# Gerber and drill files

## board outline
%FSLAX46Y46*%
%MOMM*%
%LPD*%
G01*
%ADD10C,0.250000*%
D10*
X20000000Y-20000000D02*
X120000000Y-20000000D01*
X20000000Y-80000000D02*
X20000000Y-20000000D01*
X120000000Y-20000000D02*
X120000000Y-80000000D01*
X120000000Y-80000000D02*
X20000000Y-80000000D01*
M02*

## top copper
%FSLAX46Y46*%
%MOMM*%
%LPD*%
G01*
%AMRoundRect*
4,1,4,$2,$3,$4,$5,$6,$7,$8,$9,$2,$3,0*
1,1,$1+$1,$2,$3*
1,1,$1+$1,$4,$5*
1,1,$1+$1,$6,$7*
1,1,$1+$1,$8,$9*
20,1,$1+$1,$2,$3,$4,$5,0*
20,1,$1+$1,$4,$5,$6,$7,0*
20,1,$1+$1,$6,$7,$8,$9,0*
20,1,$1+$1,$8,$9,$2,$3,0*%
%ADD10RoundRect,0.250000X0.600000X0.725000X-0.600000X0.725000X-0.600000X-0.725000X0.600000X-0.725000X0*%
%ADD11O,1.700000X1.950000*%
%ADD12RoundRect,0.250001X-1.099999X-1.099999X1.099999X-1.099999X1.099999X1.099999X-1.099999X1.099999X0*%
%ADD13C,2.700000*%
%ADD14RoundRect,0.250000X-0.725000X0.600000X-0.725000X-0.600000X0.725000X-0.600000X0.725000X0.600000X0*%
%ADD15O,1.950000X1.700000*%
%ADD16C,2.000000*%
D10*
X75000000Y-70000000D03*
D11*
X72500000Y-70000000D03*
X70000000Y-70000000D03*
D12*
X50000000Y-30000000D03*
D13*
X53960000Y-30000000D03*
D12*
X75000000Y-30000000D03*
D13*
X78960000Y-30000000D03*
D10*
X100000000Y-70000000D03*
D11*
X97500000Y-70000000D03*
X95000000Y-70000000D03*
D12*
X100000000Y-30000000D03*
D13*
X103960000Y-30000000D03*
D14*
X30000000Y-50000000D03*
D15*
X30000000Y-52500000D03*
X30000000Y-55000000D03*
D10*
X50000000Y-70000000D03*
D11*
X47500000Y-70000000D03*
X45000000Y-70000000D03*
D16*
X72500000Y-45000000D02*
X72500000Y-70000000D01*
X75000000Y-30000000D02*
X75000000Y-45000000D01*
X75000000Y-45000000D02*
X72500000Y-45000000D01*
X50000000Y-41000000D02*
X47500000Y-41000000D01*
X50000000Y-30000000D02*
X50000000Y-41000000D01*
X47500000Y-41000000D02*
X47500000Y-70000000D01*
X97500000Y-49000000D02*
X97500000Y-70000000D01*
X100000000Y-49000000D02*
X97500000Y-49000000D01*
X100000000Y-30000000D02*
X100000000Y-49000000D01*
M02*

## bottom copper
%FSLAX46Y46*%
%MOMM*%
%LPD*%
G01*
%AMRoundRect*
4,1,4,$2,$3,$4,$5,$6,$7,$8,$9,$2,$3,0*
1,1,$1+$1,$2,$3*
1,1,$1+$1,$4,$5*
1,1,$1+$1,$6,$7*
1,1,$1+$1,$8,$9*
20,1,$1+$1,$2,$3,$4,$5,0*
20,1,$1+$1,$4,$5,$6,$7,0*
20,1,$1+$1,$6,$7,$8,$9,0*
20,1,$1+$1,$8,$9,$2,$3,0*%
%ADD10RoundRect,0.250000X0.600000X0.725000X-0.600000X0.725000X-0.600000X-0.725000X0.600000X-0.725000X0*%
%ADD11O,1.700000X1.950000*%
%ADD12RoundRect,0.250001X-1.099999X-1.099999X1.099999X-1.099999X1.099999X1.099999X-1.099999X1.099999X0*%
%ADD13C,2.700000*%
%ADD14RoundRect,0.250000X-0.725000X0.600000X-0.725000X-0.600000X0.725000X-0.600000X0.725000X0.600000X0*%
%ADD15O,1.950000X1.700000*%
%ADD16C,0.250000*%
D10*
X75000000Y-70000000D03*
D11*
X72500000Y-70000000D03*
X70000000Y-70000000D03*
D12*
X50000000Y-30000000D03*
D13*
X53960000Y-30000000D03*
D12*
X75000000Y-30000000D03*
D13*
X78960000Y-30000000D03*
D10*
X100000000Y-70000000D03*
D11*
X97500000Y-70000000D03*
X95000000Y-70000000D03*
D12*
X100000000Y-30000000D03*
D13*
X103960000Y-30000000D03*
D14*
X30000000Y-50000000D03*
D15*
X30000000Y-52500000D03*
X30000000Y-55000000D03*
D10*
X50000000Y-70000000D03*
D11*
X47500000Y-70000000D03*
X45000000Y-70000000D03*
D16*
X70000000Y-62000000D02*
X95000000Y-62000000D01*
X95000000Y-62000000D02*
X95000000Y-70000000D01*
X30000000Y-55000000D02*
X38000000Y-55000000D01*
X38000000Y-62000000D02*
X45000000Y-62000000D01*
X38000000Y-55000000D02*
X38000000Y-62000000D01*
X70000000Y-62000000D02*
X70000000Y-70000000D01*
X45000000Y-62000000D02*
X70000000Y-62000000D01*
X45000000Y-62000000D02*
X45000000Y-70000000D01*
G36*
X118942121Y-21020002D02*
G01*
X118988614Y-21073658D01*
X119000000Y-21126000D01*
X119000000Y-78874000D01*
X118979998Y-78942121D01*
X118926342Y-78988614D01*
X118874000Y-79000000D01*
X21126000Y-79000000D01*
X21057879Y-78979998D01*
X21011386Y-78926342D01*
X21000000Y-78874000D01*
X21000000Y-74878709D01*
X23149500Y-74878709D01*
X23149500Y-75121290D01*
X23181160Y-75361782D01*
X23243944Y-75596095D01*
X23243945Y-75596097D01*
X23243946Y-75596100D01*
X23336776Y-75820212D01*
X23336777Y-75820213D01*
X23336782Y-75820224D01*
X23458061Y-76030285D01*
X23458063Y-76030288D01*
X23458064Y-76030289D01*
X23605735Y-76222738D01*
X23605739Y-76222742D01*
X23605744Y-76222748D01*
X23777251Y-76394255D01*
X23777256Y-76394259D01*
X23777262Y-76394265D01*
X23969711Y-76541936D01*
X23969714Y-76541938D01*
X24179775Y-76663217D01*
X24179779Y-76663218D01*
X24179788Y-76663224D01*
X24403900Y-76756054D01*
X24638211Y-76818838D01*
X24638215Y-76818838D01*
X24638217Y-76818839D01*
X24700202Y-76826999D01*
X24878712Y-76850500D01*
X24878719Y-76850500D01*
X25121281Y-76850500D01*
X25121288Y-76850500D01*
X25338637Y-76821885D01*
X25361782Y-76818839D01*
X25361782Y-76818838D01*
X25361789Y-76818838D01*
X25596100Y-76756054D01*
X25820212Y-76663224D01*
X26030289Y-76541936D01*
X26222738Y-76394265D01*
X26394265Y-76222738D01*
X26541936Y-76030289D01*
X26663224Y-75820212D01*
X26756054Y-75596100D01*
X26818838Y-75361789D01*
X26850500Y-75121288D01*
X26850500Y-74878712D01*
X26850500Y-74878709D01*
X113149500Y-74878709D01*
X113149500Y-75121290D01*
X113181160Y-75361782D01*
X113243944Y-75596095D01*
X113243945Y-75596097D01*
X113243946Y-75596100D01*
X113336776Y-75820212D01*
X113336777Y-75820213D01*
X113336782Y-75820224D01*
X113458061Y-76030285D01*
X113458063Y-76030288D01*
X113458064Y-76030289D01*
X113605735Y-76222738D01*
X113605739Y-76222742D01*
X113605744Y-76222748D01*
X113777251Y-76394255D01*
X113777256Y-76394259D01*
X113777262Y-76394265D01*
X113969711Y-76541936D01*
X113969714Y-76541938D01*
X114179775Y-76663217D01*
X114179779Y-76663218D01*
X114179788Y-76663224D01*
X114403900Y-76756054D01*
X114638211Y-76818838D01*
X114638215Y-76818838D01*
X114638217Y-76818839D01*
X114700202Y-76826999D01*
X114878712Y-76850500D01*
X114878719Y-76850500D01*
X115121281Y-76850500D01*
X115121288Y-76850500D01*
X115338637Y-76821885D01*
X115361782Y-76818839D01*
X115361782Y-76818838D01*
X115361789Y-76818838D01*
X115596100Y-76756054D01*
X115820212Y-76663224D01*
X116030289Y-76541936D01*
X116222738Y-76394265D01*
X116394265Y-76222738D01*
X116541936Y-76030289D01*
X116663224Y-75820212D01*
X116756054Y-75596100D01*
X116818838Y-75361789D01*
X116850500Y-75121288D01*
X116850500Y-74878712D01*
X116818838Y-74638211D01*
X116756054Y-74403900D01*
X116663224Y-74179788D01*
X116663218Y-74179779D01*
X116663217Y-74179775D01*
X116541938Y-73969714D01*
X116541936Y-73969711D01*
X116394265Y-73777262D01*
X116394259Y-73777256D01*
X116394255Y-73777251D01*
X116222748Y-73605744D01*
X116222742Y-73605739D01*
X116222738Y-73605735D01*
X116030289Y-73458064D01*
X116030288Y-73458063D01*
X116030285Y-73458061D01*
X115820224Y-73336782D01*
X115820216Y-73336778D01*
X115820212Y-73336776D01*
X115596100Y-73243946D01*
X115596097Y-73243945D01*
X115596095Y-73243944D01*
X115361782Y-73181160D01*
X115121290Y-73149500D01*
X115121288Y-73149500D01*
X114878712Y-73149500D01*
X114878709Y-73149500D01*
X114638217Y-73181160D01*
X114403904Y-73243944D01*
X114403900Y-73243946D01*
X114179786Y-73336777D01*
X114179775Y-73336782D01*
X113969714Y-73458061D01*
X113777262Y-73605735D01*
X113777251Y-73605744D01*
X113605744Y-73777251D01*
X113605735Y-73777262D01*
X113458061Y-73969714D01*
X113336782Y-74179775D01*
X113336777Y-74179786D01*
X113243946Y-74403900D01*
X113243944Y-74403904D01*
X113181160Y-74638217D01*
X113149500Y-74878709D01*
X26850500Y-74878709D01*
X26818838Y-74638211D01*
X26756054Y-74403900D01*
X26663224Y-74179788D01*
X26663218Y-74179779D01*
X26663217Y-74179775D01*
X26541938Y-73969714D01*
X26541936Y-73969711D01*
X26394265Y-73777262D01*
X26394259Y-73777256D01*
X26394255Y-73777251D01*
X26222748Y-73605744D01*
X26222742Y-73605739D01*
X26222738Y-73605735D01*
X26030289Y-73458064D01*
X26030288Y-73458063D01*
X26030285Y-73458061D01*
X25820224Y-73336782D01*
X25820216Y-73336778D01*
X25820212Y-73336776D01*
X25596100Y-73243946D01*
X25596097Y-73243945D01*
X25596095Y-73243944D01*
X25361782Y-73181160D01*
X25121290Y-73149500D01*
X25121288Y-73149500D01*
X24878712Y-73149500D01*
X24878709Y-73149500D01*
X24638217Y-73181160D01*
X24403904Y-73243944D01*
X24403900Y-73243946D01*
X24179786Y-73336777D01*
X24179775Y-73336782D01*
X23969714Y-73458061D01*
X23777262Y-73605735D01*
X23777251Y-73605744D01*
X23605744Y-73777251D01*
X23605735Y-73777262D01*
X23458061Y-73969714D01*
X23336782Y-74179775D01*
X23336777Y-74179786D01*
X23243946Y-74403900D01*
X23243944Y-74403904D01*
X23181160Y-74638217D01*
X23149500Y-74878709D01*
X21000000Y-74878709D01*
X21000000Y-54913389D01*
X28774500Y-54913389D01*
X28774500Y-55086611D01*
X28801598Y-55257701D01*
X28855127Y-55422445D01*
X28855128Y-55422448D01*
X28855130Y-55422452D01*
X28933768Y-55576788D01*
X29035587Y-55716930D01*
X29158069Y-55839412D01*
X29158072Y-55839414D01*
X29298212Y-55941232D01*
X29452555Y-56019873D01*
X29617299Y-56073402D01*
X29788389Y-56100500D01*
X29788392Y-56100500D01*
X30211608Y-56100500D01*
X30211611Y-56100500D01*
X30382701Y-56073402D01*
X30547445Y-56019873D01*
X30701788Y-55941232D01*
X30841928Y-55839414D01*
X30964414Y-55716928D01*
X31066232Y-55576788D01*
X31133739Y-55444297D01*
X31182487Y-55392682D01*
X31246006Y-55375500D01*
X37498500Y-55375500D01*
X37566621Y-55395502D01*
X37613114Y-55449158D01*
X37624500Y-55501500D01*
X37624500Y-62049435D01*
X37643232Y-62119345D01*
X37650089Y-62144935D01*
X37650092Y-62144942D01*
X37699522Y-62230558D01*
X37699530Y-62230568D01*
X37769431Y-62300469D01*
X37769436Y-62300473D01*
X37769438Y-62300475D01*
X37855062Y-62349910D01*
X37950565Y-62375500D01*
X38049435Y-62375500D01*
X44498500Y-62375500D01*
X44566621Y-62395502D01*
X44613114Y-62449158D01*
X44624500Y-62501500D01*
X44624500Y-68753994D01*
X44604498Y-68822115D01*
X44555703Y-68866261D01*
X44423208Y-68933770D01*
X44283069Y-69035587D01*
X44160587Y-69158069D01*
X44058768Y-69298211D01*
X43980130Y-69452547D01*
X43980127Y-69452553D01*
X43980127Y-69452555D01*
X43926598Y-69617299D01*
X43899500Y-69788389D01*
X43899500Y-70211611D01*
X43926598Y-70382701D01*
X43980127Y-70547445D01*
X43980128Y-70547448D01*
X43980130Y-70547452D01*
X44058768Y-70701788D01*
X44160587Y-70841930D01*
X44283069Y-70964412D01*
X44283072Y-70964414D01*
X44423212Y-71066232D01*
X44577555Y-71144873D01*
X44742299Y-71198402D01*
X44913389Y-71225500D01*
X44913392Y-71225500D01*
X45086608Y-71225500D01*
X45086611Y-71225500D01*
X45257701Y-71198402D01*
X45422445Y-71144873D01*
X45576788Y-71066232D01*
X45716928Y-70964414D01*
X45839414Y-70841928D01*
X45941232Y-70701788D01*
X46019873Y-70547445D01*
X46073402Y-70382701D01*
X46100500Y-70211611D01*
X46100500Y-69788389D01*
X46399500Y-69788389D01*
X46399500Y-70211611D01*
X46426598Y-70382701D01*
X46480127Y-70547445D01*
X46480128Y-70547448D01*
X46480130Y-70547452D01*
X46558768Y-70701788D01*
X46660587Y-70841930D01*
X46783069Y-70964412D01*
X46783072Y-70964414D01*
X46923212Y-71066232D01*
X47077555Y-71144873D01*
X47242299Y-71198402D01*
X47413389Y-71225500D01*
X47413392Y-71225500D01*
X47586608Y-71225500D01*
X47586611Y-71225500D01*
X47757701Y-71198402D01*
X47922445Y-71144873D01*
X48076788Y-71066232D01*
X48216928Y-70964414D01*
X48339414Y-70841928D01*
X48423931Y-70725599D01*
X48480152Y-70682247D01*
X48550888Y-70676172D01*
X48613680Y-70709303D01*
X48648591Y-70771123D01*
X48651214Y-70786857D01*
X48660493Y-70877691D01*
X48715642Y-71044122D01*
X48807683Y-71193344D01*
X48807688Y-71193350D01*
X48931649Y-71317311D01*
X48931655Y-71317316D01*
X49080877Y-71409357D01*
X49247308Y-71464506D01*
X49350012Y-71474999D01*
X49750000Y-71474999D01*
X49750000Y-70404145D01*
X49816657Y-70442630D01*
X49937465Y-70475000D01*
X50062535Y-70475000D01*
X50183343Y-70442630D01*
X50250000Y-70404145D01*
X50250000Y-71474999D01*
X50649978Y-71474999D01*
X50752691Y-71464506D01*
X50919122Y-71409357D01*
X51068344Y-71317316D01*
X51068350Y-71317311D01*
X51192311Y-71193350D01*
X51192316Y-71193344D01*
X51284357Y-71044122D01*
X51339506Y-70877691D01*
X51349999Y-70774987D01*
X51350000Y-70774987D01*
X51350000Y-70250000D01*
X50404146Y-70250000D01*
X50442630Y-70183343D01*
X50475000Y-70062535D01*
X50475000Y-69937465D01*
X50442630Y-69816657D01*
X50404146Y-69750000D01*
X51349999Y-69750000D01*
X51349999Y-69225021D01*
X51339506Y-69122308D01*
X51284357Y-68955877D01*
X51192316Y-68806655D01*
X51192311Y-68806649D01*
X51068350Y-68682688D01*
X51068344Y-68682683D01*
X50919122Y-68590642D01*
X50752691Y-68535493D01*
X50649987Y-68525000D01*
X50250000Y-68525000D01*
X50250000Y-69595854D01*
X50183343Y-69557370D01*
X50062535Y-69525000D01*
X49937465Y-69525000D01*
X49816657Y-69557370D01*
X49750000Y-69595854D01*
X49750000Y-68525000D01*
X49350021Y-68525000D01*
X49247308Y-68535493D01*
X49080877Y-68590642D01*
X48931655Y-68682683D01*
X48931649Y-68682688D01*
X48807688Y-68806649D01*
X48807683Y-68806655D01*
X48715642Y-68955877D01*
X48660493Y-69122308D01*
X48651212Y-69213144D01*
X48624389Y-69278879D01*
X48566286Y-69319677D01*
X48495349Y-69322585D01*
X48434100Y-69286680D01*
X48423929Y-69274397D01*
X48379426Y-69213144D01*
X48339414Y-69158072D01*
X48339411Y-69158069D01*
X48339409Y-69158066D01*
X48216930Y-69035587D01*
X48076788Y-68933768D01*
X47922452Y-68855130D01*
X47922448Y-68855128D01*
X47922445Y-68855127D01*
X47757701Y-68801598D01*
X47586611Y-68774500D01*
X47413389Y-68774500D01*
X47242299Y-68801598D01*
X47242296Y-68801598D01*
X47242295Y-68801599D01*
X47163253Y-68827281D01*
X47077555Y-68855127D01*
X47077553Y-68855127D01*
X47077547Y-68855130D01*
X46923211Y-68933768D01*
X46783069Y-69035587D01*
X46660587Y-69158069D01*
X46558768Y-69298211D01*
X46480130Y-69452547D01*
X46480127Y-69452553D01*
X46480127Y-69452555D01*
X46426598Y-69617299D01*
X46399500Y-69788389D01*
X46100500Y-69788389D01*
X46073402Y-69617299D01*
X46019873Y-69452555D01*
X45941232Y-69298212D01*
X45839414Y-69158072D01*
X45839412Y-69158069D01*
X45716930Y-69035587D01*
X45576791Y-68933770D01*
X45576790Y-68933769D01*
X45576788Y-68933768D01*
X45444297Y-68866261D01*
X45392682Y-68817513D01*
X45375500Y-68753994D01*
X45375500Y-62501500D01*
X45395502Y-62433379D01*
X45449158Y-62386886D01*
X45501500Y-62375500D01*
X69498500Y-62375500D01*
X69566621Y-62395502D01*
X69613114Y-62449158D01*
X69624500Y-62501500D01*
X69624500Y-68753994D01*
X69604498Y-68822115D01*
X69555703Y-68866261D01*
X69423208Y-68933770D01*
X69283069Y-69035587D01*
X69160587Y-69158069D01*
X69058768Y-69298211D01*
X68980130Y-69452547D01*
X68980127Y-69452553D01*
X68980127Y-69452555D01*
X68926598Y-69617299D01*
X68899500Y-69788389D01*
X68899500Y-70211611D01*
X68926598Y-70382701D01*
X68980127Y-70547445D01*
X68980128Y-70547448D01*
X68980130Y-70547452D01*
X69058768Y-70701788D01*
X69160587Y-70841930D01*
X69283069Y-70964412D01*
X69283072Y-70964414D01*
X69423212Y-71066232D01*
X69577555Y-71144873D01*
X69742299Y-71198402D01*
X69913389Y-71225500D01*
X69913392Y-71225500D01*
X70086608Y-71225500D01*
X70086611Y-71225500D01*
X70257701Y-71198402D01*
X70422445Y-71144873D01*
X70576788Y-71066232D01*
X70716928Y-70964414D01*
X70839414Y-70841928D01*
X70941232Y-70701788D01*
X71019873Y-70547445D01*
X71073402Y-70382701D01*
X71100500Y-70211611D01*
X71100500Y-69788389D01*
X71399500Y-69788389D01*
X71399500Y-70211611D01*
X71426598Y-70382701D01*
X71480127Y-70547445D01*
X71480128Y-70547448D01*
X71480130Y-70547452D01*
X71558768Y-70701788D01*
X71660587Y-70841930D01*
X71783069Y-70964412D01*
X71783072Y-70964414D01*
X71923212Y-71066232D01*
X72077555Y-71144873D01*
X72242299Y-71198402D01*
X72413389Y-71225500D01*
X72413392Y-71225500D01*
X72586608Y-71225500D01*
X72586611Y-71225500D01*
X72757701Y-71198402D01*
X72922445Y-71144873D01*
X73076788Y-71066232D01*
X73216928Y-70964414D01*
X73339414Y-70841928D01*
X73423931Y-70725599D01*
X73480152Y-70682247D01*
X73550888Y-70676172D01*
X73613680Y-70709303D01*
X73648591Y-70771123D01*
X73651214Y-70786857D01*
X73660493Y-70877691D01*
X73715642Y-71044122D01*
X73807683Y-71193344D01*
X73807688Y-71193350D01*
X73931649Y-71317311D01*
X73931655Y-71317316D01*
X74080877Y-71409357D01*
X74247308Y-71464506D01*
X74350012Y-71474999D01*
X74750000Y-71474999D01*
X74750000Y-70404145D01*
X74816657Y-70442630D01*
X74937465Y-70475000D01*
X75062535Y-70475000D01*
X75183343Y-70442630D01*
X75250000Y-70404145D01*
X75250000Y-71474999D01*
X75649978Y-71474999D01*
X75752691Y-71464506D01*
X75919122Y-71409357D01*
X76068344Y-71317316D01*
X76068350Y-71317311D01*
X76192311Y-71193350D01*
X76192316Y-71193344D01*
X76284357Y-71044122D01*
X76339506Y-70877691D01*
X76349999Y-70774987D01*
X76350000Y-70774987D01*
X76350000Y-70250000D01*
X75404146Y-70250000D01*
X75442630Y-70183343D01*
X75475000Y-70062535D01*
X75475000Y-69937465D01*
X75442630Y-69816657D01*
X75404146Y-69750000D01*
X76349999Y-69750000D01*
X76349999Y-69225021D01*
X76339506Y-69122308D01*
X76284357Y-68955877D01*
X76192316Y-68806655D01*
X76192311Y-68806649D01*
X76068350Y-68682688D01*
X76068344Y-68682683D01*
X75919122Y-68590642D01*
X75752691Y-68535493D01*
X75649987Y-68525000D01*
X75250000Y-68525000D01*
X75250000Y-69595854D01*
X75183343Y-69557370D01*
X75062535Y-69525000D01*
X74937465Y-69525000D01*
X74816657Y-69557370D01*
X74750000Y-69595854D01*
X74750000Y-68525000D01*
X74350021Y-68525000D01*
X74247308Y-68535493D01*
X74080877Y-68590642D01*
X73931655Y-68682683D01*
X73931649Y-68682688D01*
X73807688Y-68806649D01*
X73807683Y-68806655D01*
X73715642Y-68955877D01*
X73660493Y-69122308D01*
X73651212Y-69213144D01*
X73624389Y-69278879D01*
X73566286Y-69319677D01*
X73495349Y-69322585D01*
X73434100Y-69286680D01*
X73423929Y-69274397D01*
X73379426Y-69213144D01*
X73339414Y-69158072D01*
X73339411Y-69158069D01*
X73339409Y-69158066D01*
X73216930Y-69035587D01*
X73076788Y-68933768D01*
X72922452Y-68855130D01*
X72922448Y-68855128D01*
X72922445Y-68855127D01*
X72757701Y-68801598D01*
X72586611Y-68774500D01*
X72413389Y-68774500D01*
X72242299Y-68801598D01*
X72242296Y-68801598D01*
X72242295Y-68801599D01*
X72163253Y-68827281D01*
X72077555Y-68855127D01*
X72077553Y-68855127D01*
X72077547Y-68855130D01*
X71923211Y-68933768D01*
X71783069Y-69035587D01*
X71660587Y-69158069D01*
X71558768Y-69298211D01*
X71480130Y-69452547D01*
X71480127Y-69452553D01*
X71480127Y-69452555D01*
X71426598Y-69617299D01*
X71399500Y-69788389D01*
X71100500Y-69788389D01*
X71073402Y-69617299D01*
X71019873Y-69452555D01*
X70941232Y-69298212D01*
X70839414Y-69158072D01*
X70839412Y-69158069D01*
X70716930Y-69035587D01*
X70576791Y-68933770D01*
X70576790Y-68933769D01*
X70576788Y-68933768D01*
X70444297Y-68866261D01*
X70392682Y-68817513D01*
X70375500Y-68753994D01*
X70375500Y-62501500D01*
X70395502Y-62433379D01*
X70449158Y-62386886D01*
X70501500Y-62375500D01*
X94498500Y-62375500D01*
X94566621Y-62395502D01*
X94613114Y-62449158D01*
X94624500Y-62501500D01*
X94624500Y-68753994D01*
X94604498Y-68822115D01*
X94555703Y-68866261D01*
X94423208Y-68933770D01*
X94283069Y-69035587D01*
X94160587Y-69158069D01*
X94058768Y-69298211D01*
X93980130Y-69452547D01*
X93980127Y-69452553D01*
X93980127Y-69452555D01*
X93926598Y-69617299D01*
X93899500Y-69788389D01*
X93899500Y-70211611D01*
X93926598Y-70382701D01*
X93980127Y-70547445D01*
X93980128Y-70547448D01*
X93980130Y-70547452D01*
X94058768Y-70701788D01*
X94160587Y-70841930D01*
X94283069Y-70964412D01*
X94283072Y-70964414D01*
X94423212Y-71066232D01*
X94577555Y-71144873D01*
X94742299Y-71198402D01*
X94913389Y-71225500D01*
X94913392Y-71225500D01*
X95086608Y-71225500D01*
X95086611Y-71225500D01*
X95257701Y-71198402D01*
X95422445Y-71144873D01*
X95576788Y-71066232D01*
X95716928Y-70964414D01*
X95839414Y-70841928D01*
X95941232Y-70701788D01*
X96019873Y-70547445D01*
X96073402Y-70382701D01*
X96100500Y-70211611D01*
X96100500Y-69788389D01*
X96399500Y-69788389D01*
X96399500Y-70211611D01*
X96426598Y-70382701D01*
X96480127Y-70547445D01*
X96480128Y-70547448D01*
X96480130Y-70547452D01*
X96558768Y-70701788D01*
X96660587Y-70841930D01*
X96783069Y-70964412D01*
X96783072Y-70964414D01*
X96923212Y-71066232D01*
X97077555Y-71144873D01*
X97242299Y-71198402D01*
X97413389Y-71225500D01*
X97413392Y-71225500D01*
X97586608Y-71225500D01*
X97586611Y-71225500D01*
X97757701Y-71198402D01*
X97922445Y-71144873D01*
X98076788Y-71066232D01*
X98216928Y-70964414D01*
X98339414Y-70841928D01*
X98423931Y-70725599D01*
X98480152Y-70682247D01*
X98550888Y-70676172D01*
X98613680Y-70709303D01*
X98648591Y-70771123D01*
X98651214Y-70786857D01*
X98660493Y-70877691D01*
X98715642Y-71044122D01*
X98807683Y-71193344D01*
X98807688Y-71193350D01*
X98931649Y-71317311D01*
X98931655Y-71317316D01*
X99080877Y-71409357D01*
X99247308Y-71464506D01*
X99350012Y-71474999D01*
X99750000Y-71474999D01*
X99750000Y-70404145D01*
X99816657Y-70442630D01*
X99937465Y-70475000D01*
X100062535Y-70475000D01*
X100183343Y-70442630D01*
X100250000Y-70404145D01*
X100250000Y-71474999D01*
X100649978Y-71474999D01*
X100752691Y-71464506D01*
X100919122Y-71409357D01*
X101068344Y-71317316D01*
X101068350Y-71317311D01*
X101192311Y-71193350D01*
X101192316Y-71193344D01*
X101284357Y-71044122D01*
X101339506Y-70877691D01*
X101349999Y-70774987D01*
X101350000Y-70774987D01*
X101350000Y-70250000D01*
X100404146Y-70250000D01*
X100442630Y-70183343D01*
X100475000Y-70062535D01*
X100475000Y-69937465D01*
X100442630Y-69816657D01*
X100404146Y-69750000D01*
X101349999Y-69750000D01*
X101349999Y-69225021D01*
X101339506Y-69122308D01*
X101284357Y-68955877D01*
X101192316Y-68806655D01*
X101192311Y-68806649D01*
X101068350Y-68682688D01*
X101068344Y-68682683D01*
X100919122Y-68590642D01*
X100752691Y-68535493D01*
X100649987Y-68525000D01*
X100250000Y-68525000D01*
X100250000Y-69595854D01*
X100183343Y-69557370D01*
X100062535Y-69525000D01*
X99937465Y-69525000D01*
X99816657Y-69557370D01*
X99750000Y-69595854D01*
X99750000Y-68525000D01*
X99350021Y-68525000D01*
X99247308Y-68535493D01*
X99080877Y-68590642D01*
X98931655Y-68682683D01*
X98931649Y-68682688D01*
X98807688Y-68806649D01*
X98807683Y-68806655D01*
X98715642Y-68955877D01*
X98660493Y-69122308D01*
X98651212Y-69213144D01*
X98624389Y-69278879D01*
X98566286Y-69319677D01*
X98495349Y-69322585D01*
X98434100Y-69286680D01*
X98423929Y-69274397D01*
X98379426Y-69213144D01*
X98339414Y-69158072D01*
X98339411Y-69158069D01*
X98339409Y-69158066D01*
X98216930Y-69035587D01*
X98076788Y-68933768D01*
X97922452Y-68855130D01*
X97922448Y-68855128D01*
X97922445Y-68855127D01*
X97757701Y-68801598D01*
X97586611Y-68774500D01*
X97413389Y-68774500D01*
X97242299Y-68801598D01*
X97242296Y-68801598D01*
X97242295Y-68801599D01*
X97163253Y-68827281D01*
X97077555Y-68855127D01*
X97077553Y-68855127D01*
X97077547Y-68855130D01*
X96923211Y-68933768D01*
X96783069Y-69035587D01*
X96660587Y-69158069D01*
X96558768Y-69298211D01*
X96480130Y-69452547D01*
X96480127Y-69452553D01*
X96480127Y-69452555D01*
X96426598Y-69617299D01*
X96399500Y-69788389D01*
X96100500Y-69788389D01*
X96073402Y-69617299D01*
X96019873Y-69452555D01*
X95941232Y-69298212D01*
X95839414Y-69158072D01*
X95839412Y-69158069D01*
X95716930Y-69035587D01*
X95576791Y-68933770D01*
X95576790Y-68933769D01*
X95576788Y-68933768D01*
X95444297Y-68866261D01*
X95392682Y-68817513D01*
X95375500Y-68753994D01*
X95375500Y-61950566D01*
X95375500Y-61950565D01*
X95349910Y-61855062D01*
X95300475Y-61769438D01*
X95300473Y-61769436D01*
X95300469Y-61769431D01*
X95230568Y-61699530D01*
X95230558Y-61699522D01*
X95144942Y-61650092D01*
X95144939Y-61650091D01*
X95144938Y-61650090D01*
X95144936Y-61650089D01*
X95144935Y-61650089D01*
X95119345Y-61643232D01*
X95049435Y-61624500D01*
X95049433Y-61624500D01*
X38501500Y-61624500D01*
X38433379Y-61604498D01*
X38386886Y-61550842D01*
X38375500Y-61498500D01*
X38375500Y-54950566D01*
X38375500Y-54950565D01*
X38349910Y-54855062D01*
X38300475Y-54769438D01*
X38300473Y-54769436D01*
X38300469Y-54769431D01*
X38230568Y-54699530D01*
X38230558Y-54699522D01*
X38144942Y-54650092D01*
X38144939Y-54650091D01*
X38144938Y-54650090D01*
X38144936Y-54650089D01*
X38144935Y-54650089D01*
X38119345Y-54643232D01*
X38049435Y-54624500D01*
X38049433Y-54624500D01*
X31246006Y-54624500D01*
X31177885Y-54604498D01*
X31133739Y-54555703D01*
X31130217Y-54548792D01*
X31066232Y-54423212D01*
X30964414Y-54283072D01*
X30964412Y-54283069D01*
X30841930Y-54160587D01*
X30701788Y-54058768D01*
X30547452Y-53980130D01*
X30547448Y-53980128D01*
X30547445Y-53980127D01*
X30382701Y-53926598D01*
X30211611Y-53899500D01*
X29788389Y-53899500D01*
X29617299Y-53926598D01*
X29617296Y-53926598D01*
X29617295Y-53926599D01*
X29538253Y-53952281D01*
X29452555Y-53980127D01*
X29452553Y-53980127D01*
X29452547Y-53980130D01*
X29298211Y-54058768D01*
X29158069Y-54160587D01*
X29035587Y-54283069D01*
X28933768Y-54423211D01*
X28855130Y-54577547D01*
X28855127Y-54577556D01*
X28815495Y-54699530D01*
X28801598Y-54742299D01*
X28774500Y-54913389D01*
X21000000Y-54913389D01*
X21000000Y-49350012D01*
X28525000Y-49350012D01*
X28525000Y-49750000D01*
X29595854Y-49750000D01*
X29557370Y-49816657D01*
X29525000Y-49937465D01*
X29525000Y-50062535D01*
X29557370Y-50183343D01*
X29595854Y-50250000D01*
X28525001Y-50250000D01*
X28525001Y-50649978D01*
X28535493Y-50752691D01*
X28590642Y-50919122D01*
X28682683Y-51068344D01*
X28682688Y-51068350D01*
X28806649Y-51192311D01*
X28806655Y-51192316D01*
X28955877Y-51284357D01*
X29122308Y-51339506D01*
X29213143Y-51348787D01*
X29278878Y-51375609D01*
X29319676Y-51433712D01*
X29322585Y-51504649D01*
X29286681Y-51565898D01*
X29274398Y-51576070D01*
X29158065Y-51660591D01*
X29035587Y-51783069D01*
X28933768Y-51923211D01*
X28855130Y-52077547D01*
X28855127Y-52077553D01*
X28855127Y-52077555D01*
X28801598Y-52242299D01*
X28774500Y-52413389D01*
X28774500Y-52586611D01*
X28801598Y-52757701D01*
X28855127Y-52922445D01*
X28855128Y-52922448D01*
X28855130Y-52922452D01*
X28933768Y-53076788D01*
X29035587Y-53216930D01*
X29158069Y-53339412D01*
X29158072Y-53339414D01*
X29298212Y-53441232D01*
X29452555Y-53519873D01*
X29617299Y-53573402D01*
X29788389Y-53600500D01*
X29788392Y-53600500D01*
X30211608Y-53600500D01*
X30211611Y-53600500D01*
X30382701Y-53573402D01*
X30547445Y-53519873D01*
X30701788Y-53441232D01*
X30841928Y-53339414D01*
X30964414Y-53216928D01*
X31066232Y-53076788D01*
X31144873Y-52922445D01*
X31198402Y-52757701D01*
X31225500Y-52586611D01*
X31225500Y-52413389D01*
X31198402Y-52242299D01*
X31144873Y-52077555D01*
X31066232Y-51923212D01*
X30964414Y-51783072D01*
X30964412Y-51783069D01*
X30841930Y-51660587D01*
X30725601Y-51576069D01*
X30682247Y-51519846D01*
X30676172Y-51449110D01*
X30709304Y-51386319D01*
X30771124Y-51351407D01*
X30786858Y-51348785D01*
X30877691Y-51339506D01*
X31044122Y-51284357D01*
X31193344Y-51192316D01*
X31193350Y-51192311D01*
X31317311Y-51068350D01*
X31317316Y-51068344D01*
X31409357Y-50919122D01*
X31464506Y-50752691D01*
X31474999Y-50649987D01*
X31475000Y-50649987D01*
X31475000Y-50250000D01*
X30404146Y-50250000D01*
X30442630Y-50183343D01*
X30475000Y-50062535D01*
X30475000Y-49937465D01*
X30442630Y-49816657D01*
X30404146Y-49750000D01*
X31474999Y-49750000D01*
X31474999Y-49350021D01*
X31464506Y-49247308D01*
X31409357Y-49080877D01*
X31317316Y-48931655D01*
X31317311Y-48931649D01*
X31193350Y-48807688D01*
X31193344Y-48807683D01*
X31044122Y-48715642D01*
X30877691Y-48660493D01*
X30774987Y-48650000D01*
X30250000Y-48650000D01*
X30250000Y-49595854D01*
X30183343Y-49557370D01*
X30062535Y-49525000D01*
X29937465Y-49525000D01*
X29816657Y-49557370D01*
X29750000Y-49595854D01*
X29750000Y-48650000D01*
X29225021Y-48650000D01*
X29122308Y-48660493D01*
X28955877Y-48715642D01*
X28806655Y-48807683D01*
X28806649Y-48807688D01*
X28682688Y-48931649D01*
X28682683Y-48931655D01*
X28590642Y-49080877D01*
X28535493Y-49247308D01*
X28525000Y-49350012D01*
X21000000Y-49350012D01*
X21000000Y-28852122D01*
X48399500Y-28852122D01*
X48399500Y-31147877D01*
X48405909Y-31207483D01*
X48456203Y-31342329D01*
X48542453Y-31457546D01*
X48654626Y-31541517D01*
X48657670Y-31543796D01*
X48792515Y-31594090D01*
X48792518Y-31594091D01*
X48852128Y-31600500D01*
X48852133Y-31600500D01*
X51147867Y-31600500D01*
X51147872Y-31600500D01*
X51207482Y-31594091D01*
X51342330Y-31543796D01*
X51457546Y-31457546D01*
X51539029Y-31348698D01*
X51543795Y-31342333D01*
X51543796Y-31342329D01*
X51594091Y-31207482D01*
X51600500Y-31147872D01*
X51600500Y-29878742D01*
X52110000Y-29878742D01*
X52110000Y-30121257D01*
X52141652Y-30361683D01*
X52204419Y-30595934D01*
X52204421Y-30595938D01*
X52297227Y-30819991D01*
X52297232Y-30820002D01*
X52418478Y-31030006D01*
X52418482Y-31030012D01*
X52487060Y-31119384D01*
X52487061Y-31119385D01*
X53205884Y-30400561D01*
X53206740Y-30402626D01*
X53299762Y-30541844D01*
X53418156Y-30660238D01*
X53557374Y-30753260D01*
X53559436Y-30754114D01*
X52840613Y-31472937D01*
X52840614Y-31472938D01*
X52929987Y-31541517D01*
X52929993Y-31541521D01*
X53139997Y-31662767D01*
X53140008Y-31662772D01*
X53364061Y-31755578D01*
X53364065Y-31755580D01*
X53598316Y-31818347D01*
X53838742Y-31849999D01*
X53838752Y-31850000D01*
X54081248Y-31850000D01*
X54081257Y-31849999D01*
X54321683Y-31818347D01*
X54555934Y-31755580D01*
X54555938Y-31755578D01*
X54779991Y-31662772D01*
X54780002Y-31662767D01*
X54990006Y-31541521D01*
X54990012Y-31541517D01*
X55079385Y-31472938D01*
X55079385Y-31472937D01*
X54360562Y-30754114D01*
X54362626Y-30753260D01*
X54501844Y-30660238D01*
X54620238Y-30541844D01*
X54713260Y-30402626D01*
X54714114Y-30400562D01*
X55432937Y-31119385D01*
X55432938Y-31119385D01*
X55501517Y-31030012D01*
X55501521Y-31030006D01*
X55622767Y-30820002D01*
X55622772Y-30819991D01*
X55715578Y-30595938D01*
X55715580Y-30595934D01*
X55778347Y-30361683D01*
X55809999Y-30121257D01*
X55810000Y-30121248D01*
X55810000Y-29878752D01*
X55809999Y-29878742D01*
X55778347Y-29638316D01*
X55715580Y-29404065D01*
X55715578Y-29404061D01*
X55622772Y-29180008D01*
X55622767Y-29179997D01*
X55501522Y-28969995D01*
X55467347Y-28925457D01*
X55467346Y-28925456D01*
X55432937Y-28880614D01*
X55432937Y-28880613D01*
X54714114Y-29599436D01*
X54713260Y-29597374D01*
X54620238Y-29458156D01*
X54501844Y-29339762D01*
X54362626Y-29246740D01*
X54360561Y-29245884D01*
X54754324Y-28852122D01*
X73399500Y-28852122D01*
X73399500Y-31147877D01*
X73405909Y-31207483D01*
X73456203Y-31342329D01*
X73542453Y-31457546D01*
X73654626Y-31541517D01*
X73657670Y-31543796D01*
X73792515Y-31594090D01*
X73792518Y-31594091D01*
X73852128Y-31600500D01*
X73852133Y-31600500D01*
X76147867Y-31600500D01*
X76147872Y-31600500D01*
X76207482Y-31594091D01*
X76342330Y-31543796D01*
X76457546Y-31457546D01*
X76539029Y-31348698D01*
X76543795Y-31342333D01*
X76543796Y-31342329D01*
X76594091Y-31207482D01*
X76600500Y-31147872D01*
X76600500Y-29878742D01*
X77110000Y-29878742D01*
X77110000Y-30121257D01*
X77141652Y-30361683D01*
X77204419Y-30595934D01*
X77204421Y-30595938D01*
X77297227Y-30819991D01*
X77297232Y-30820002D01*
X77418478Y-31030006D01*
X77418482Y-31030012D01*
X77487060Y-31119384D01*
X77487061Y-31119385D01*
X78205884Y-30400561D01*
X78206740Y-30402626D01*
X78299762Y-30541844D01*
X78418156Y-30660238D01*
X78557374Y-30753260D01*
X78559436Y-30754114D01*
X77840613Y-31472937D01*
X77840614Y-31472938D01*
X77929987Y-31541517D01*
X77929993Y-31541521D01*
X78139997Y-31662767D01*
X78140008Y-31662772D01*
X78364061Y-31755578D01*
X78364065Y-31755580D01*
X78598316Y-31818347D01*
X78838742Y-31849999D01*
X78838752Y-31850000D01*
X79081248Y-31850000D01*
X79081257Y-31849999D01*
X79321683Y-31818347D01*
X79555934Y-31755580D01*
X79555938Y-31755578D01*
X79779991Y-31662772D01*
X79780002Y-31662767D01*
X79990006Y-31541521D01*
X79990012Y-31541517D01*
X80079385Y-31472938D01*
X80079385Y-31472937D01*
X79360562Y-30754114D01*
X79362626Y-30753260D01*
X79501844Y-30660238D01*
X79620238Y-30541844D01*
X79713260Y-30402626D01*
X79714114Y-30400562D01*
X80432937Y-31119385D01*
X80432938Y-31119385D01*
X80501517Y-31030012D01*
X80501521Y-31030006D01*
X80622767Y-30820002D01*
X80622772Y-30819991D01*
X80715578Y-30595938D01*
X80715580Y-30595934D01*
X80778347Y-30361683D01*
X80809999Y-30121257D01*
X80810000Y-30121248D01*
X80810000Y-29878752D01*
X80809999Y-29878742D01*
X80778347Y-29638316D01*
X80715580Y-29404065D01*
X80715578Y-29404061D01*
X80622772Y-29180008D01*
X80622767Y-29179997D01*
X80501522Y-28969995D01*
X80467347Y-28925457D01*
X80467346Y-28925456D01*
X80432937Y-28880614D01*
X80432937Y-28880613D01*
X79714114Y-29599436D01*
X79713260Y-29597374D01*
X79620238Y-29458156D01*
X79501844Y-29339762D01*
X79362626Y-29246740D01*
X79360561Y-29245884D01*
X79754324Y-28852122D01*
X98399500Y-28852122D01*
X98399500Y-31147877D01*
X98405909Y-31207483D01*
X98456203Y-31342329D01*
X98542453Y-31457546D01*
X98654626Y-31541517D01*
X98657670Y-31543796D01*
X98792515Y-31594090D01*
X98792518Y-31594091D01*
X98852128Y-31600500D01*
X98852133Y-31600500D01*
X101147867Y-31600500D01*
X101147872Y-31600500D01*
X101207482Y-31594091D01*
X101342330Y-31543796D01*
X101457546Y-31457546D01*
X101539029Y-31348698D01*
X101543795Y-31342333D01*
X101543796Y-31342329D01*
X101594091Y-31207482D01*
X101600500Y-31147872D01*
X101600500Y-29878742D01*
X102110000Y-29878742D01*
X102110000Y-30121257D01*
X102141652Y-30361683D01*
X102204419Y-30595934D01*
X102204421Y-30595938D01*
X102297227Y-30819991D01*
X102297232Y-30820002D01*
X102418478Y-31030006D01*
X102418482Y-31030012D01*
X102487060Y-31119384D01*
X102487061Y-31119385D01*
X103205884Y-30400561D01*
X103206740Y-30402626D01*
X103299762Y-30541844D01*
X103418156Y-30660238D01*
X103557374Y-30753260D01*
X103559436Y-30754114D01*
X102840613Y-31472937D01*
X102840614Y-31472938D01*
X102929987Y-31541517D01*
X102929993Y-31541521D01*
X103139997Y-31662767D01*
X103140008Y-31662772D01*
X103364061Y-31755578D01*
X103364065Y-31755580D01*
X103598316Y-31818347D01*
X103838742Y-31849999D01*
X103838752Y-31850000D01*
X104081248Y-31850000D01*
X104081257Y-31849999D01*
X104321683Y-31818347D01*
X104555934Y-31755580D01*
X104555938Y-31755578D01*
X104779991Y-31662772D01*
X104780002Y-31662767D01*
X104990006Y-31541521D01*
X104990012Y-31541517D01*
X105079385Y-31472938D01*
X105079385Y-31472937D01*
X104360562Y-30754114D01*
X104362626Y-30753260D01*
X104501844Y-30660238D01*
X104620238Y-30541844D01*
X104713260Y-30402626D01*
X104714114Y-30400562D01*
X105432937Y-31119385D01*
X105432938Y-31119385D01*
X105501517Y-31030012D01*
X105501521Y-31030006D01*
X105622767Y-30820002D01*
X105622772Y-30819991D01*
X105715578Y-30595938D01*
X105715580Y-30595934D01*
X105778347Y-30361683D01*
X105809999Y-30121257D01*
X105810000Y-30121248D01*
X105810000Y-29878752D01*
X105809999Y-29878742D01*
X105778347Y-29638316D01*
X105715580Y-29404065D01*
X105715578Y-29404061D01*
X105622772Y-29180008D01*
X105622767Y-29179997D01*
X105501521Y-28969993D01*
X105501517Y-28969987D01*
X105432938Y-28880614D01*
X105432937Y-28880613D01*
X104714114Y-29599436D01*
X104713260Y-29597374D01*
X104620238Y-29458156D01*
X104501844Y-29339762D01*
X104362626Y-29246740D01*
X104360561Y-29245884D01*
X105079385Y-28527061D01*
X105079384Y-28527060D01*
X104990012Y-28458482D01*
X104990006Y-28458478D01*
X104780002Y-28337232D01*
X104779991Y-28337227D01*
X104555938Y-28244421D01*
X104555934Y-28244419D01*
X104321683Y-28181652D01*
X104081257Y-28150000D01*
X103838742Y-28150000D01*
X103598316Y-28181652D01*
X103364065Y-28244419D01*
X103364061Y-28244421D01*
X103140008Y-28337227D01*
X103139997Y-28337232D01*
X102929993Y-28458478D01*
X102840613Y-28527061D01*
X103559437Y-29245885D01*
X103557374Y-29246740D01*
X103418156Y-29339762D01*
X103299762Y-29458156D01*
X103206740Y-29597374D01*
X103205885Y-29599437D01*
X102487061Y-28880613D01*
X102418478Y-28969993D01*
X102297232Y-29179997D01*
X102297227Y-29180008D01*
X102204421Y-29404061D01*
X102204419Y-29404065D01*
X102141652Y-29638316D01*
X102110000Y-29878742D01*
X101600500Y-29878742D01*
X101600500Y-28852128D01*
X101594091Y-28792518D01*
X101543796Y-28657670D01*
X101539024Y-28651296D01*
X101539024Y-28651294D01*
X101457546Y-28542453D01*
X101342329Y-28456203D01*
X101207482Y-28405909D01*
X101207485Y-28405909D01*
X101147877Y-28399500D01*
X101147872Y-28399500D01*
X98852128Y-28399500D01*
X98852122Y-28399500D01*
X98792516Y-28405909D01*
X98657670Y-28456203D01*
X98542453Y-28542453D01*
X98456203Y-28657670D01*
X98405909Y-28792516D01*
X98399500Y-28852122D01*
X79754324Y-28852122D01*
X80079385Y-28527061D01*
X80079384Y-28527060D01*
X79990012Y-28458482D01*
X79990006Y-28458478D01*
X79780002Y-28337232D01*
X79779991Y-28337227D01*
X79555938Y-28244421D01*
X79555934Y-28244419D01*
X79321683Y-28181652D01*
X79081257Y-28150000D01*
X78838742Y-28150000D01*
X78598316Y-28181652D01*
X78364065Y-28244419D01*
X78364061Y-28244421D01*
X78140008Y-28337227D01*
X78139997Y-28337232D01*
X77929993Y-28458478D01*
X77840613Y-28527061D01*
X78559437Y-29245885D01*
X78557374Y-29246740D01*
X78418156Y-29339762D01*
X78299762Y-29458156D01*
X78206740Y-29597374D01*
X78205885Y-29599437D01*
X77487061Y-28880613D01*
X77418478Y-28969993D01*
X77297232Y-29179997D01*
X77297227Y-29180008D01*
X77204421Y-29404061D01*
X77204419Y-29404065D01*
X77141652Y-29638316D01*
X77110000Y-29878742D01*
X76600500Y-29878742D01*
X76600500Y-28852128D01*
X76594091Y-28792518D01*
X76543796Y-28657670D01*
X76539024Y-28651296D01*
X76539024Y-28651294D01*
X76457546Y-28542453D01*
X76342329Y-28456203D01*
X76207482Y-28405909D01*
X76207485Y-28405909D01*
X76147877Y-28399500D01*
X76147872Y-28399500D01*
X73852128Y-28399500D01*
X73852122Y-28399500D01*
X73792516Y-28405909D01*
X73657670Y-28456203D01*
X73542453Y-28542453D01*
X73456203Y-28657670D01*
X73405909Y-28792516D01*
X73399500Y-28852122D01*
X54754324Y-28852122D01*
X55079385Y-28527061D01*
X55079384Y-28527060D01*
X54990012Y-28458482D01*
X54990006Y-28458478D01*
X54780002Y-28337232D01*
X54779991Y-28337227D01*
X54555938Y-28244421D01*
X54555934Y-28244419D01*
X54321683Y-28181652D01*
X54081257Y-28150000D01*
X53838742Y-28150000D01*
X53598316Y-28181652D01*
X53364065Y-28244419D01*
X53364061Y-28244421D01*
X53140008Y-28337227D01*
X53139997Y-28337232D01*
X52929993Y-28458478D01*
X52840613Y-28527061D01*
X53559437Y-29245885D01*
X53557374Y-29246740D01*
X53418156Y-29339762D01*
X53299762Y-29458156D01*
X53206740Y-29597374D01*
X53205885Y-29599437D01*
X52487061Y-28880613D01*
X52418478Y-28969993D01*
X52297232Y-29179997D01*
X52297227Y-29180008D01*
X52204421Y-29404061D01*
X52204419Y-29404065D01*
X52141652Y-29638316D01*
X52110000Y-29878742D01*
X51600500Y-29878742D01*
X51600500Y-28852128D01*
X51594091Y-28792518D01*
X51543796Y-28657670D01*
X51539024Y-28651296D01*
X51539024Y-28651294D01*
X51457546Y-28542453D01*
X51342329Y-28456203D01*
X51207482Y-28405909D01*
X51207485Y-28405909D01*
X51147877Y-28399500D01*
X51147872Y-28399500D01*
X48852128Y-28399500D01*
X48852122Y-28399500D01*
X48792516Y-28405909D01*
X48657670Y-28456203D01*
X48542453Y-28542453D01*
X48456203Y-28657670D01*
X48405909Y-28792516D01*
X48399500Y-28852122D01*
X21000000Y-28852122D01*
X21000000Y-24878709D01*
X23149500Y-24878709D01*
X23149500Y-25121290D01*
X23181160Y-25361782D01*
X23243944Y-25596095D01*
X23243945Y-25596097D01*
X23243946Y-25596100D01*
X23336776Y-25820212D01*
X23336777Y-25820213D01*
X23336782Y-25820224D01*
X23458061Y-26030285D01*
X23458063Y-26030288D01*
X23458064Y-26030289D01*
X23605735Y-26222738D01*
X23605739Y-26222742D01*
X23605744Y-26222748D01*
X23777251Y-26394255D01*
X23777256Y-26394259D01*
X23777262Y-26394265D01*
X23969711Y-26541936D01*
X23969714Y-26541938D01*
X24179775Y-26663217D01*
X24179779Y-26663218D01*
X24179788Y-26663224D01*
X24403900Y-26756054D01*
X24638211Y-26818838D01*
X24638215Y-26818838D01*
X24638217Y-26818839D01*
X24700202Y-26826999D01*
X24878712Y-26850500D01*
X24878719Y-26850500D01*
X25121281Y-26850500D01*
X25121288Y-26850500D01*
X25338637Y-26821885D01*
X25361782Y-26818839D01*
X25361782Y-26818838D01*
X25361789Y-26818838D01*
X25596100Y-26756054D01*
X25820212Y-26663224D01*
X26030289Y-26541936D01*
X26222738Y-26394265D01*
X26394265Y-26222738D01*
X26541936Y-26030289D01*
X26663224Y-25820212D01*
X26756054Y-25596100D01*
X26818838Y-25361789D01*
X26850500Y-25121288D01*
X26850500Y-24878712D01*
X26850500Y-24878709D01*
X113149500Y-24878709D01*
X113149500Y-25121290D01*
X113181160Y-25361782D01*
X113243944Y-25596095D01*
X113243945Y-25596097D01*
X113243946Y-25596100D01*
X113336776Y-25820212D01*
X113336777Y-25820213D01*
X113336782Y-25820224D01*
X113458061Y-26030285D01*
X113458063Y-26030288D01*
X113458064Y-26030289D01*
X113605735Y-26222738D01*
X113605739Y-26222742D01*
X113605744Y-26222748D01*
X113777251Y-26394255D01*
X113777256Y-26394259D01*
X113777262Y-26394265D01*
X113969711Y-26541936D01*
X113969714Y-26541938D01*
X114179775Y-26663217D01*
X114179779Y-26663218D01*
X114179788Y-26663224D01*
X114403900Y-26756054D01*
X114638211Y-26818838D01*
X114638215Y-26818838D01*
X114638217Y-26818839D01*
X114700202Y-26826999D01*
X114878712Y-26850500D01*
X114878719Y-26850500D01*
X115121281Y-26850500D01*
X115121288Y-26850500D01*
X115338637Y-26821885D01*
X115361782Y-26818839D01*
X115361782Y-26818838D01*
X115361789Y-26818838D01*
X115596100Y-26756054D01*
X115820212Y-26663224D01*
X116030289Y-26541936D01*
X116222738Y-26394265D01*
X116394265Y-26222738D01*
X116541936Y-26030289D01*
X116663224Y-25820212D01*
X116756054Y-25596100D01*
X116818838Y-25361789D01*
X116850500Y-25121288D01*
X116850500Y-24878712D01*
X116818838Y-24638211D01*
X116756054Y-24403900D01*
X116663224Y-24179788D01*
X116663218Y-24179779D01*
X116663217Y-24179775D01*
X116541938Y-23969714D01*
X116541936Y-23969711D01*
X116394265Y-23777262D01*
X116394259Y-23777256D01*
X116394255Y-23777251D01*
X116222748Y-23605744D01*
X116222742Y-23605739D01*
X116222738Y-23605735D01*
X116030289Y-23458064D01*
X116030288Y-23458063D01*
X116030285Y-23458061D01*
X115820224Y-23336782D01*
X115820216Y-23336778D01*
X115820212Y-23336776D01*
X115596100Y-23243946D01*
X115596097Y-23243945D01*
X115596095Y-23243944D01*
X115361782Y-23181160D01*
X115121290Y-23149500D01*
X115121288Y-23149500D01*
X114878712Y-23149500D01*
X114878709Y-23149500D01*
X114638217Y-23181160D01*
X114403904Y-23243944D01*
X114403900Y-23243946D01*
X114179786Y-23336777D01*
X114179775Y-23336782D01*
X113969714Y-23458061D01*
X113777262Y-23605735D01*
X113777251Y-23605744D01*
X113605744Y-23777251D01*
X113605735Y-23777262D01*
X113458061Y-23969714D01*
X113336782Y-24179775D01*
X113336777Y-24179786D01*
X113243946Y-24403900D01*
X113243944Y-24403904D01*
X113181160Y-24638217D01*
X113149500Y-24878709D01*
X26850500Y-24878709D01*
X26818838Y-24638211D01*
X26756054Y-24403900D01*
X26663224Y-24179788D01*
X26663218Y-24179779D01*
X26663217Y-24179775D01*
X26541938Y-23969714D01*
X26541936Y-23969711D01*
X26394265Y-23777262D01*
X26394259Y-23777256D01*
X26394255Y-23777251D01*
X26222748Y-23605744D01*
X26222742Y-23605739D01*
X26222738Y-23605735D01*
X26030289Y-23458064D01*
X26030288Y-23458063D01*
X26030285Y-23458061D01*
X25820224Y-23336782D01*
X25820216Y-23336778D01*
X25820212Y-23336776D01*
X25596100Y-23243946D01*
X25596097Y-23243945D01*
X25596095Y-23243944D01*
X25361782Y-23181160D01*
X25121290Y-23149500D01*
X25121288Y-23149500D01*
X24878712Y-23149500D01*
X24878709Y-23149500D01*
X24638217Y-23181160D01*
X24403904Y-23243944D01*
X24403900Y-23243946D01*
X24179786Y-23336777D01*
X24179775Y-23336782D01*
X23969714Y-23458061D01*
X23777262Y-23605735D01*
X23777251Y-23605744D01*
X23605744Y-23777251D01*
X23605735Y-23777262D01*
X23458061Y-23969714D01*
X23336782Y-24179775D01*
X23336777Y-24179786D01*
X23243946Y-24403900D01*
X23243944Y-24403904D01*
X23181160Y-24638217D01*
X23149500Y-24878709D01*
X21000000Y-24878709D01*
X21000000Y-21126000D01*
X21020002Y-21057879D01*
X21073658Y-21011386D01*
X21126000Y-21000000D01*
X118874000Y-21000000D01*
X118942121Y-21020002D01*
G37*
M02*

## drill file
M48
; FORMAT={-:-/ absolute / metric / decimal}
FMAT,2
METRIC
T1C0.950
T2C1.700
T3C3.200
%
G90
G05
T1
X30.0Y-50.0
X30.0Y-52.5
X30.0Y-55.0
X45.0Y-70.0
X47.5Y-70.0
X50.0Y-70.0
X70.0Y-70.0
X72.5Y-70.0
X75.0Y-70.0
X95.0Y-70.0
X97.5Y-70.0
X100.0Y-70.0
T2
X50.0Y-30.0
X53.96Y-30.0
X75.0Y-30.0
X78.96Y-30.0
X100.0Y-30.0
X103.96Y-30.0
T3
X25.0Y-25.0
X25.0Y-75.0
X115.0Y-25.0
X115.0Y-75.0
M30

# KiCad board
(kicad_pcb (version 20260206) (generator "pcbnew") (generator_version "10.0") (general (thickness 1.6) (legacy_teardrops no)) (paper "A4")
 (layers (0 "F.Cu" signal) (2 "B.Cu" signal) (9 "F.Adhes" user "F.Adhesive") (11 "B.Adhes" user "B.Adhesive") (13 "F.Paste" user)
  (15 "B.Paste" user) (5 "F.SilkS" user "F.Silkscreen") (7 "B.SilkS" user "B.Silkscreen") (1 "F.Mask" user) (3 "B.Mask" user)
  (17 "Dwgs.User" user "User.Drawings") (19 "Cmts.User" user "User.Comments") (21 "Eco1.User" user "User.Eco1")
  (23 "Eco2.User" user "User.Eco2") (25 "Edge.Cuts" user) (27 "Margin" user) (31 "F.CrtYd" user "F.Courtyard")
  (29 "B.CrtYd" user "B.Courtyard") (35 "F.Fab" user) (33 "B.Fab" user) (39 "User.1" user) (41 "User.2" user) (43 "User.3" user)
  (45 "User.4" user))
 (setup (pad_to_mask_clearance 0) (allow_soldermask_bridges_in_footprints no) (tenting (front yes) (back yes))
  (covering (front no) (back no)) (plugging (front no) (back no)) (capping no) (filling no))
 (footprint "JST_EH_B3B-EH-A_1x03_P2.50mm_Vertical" (layer "F.Cu") (at 75 70 180)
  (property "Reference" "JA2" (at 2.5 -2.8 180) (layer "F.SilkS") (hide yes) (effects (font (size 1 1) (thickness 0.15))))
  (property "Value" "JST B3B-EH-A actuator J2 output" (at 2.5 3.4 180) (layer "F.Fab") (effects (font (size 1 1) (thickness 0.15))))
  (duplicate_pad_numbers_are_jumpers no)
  (pad "1" thru_hole roundrect (at 0 0 180) (size 1.7 1.95) (drill 0.95) (layers "*.Cu" "*.Mask") (remove_unused_layers no)
   (roundrect_rratio 0.147059) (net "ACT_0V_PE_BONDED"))
  (pad "2" thru_hole oval (at 2.5 0 180) (size 1.7 1.95) (drill 0.95) (layers "*.Cu" "*.Mask") (remove_unused_layers no)
   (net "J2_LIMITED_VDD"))
  (pad "3" thru_hole oval (at 5 0 180) (size 1.7 1.95) (drill 0.95) (layers "*.Cu" "*.Mask") (remove_unused_layers no) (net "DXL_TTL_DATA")))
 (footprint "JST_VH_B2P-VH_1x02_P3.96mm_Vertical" (layer "F.Cu") (at 50 30)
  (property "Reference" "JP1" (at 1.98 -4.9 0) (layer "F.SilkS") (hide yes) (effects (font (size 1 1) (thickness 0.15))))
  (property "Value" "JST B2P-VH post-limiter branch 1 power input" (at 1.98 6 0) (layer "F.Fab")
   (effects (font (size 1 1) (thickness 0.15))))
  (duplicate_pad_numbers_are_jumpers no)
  (pad "1" thru_hole roundrect (at 0 0) (size 2.7 2.7) (drill 1.7) (layers "*.Cu" "*.Mask") (remove_unused_layers no)
   (roundrect_rratio 0.092593) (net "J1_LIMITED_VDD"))
  (pad "2" thru_hole circle (at 3.96 0) (size 2.7 2.7) (drill 1.7) (layers "*.Cu" "*.Mask") (remove_unused_layers no)
   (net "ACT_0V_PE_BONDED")))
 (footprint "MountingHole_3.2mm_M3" (layer "F.Cu") (at 115 75)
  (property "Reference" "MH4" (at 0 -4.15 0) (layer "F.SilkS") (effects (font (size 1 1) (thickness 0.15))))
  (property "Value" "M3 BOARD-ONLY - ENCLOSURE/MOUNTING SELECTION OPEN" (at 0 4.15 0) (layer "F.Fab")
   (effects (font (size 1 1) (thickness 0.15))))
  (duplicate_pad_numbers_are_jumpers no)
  (pad "" np_thru_hole circle (at 0 0) (size 3.2 3.2) (drill 3.2) (layers "*.Cu" "*.Mask")))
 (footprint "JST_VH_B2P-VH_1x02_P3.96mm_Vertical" (layer "F.Cu") (at 75 30)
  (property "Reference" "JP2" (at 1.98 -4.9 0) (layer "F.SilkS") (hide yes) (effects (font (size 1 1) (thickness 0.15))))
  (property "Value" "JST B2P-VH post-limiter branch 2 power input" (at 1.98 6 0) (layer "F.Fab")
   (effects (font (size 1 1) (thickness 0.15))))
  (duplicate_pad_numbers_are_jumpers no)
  (pad "1" thru_hole roundrect (at 0 0) (size 2.7 2.7) (drill 1.7) (layers "*.Cu" "*.Mask") (remove_unused_layers no)
   (roundrect_rratio 0.092593) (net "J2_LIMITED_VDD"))
  (pad "2" thru_hole circle (at 3.96 0) (size 2.7 2.7) (drill 1.7) (layers "*.Cu" "*.Mask") (remove_unused_layers no)
   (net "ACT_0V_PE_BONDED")))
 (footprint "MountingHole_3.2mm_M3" (layer "F.Cu") (at 25 25)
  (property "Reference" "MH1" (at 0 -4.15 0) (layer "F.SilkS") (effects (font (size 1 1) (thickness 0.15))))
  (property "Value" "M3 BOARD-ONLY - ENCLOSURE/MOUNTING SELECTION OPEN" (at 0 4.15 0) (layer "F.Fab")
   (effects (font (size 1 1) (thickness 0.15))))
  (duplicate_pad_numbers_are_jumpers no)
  (pad "" np_thru_hole circle (at 0 0) (size 3.2 3.2) (drill 3.2) (layers "*.Cu" "*.Mask")))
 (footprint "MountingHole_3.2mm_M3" (layer "F.Cu") (at 115 25)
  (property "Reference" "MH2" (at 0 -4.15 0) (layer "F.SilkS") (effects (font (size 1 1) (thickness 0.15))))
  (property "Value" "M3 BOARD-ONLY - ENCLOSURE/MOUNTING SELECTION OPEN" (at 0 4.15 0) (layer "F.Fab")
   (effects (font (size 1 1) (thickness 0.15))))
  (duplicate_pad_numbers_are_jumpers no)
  (pad "" np_thru_hole circle (at 0 0) (size 3.2 3.2) (drill 3.2) (layers "*.Cu" "*.Mask")))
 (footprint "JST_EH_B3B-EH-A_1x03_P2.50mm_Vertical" (layer "F.Cu") (at 100 70 180)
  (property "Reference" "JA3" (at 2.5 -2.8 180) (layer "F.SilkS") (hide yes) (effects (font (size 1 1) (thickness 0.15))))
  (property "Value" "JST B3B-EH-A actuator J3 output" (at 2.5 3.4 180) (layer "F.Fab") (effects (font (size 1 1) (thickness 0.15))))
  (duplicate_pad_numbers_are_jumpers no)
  (pad "1" thru_hole roundrect (at 0 0 180) (size 1.7 1.95) (drill 0.95) (layers "*.Cu" "*.Mask") (remove_unused_layers no)
   (roundrect_rratio 0.147059) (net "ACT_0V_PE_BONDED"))
  (pad "2" thru_hole oval (at 2.5 0 180) (size 1.7 1.95) (drill 0.95) (layers "*.Cu" "*.Mask") (remove_unused_layers no)
   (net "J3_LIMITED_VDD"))
  (pad "3" thru_hole oval (at 5 0 180) (size 1.7 1.95) (drill 0.95) (layers "*.Cu" "*.Mask") (remove_unused_layers no) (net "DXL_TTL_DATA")))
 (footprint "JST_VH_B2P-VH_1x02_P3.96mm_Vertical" (layer "F.Cu") (at 100 30)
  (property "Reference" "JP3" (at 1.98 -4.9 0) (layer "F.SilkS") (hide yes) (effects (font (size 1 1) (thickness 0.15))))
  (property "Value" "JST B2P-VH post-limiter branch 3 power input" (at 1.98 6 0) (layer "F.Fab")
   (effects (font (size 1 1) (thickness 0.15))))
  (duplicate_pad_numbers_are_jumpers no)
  (pad "1" thru_hole roundrect (at 0 0) (size 2.7 2.7) (drill 1.7) (layers "*.Cu" "*.Mask") (remove_unused_layers no)
   (roundrect_rratio 0.092593) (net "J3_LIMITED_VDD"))
  (pad "2" thru_hole circle (at 3.96 0) (size 2.7 2.7) (drill 1.7) (layers "*.Cu" "*.Mask") (remove_unused_layers no)
   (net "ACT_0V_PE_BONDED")))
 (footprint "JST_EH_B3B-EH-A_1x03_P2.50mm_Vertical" (layer "F.Cu") (at 30 50 -90)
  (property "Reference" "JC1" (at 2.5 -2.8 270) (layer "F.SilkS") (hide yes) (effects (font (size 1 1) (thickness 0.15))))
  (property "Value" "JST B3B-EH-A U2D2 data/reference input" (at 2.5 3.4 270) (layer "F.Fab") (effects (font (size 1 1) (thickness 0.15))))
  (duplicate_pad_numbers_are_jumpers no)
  (pad "1" thru_hole roundrect (at 0 0 270) (size 1.7 1.95) (drill 0.95) (layers "*.Cu" "*.Mask") (remove_unused_layers no)
   (roundrect_rratio 0.147059) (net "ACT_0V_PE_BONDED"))
  (pad "2" thru_hole oval (at 2.5 0 270) (size 1.7 1.95) (drill 0.95) (layers "*.Cu" "*.Mask") (remove_unused_layers no))
  (pad "3" thru_hole oval (at 5 0 270) (size 1.7 1.95) (drill 0.95) (layers "*.Cu" "*.Mask") (remove_unused_layers no) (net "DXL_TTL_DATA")))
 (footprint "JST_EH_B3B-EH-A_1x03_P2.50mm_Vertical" (layer "F.Cu") (at 50 70 180)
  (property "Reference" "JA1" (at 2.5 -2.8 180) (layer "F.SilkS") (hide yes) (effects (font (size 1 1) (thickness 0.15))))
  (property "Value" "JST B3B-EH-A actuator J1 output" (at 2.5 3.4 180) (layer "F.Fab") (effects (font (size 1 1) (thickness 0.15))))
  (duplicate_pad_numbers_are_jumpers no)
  (pad "1" thru_hole roundrect (at 0 0 180) (size 1.7 1.95) (drill 0.95) (layers "*.Cu" "*.Mask") (remove_unused_layers no)
   (roundrect_rratio 0.147059) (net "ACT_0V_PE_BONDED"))
  (pad "2" thru_hole oval (at 2.5 0 180) (size 1.7 1.95) (drill 0.95) (layers "*.Cu" "*.Mask") (remove_unused_layers no)
   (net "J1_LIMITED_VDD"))
  (pad "3" thru_hole oval (at 5 0 180) (size 1.7 1.95) (drill 0.95) (layers "*.Cu" "*.Mask") (remove_unused_layers no) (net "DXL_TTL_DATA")))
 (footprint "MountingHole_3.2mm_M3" (layer "F.Cu") (at 25 75)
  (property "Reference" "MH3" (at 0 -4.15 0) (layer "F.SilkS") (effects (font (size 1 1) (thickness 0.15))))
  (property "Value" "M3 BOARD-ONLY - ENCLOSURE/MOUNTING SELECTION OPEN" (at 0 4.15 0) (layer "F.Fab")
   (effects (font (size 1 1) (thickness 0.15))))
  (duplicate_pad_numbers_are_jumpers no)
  (pad "" np_thru_hole circle (at 0 0) (size 3.2 3.2) (drill 3.2) (layers "*.Cu" "*.Mask")))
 (gr_line (start 20 20) (end 120 20) (stroke (width 0.25) (type default)) (layer "Edge.Cuts"))
 (gr_line (start 20 80) (end 20 20) (stroke (width 0.25) (type default)) (layer "Edge.Cuts"))
 (gr_line (start 120 20) (end 120 80) (stroke (width 0.25) (type default)) (layer "Edge.Cuts"))
 (gr_line (start 120 80) (end 20 80) (stroke (width 0.25) (type default)) (layer "Edge.Cuts"))
 (segment (start 72.5 45) (end 72.5 70) (width 2) (layer "F.Cu") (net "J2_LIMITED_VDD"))
 (segment (start 75 30) (end 75 45) (width 2) (layer "F.Cu") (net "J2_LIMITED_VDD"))
 (segment (start 75 45) (end 72.5 45) (width 2) (layer "F.Cu") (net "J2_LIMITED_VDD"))
 (segment (start 70 62) (end 95 62) (width 0.25) (layer "B.Cu") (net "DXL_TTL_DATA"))
 (segment (start 95 62) (end 95 70) (width 0.25) (layer "B.Cu") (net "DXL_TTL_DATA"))
 (segment (start 30 55) (end 38 55) (width 0.25) (layer "B.Cu") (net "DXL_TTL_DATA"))
 (segment (start 38 62) (end 45 62) (width 0.25) (layer "B.Cu") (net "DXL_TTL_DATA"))
 (segment (start 38 55) (end 38 62) (width 0.25) (layer "B.Cu") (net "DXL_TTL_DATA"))
 (segment (start 70 62) (end 70 70) (width 0.25) (layer "B.Cu") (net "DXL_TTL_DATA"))
 (segment (start 45 62) (end 70 62) (width 0.25) (layer "B.Cu") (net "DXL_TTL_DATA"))
 (segment (start 45 62) (end 45 70) (width 0.25) (layer "B.Cu") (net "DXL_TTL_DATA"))
 (segment (start 50 41) (end 47.5 41) (width 2) (layer "F.Cu") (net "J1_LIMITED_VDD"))
 (segment (start 50 30) (end 50 41) (width 2) (layer "F.Cu") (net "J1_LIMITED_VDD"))
 (segment (start 47.5 41) (end 47.5 70) (width 2) (layer "F.Cu") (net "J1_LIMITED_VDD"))
 (segment (start 97.5 49) (end 97.5 70) (width 2) (layer "F.Cu") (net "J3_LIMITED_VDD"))
 (segment (start 100 49) (end 97.5 49) (width 2) (layer "F.Cu") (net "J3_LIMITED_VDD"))
 (segment (start 100 30) (end 100 49) (width 2) (layer "F.Cu") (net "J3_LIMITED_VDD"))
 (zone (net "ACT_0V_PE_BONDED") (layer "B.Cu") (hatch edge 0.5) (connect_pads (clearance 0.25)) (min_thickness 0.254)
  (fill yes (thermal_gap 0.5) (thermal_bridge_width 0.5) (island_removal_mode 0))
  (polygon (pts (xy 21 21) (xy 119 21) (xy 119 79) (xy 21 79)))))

